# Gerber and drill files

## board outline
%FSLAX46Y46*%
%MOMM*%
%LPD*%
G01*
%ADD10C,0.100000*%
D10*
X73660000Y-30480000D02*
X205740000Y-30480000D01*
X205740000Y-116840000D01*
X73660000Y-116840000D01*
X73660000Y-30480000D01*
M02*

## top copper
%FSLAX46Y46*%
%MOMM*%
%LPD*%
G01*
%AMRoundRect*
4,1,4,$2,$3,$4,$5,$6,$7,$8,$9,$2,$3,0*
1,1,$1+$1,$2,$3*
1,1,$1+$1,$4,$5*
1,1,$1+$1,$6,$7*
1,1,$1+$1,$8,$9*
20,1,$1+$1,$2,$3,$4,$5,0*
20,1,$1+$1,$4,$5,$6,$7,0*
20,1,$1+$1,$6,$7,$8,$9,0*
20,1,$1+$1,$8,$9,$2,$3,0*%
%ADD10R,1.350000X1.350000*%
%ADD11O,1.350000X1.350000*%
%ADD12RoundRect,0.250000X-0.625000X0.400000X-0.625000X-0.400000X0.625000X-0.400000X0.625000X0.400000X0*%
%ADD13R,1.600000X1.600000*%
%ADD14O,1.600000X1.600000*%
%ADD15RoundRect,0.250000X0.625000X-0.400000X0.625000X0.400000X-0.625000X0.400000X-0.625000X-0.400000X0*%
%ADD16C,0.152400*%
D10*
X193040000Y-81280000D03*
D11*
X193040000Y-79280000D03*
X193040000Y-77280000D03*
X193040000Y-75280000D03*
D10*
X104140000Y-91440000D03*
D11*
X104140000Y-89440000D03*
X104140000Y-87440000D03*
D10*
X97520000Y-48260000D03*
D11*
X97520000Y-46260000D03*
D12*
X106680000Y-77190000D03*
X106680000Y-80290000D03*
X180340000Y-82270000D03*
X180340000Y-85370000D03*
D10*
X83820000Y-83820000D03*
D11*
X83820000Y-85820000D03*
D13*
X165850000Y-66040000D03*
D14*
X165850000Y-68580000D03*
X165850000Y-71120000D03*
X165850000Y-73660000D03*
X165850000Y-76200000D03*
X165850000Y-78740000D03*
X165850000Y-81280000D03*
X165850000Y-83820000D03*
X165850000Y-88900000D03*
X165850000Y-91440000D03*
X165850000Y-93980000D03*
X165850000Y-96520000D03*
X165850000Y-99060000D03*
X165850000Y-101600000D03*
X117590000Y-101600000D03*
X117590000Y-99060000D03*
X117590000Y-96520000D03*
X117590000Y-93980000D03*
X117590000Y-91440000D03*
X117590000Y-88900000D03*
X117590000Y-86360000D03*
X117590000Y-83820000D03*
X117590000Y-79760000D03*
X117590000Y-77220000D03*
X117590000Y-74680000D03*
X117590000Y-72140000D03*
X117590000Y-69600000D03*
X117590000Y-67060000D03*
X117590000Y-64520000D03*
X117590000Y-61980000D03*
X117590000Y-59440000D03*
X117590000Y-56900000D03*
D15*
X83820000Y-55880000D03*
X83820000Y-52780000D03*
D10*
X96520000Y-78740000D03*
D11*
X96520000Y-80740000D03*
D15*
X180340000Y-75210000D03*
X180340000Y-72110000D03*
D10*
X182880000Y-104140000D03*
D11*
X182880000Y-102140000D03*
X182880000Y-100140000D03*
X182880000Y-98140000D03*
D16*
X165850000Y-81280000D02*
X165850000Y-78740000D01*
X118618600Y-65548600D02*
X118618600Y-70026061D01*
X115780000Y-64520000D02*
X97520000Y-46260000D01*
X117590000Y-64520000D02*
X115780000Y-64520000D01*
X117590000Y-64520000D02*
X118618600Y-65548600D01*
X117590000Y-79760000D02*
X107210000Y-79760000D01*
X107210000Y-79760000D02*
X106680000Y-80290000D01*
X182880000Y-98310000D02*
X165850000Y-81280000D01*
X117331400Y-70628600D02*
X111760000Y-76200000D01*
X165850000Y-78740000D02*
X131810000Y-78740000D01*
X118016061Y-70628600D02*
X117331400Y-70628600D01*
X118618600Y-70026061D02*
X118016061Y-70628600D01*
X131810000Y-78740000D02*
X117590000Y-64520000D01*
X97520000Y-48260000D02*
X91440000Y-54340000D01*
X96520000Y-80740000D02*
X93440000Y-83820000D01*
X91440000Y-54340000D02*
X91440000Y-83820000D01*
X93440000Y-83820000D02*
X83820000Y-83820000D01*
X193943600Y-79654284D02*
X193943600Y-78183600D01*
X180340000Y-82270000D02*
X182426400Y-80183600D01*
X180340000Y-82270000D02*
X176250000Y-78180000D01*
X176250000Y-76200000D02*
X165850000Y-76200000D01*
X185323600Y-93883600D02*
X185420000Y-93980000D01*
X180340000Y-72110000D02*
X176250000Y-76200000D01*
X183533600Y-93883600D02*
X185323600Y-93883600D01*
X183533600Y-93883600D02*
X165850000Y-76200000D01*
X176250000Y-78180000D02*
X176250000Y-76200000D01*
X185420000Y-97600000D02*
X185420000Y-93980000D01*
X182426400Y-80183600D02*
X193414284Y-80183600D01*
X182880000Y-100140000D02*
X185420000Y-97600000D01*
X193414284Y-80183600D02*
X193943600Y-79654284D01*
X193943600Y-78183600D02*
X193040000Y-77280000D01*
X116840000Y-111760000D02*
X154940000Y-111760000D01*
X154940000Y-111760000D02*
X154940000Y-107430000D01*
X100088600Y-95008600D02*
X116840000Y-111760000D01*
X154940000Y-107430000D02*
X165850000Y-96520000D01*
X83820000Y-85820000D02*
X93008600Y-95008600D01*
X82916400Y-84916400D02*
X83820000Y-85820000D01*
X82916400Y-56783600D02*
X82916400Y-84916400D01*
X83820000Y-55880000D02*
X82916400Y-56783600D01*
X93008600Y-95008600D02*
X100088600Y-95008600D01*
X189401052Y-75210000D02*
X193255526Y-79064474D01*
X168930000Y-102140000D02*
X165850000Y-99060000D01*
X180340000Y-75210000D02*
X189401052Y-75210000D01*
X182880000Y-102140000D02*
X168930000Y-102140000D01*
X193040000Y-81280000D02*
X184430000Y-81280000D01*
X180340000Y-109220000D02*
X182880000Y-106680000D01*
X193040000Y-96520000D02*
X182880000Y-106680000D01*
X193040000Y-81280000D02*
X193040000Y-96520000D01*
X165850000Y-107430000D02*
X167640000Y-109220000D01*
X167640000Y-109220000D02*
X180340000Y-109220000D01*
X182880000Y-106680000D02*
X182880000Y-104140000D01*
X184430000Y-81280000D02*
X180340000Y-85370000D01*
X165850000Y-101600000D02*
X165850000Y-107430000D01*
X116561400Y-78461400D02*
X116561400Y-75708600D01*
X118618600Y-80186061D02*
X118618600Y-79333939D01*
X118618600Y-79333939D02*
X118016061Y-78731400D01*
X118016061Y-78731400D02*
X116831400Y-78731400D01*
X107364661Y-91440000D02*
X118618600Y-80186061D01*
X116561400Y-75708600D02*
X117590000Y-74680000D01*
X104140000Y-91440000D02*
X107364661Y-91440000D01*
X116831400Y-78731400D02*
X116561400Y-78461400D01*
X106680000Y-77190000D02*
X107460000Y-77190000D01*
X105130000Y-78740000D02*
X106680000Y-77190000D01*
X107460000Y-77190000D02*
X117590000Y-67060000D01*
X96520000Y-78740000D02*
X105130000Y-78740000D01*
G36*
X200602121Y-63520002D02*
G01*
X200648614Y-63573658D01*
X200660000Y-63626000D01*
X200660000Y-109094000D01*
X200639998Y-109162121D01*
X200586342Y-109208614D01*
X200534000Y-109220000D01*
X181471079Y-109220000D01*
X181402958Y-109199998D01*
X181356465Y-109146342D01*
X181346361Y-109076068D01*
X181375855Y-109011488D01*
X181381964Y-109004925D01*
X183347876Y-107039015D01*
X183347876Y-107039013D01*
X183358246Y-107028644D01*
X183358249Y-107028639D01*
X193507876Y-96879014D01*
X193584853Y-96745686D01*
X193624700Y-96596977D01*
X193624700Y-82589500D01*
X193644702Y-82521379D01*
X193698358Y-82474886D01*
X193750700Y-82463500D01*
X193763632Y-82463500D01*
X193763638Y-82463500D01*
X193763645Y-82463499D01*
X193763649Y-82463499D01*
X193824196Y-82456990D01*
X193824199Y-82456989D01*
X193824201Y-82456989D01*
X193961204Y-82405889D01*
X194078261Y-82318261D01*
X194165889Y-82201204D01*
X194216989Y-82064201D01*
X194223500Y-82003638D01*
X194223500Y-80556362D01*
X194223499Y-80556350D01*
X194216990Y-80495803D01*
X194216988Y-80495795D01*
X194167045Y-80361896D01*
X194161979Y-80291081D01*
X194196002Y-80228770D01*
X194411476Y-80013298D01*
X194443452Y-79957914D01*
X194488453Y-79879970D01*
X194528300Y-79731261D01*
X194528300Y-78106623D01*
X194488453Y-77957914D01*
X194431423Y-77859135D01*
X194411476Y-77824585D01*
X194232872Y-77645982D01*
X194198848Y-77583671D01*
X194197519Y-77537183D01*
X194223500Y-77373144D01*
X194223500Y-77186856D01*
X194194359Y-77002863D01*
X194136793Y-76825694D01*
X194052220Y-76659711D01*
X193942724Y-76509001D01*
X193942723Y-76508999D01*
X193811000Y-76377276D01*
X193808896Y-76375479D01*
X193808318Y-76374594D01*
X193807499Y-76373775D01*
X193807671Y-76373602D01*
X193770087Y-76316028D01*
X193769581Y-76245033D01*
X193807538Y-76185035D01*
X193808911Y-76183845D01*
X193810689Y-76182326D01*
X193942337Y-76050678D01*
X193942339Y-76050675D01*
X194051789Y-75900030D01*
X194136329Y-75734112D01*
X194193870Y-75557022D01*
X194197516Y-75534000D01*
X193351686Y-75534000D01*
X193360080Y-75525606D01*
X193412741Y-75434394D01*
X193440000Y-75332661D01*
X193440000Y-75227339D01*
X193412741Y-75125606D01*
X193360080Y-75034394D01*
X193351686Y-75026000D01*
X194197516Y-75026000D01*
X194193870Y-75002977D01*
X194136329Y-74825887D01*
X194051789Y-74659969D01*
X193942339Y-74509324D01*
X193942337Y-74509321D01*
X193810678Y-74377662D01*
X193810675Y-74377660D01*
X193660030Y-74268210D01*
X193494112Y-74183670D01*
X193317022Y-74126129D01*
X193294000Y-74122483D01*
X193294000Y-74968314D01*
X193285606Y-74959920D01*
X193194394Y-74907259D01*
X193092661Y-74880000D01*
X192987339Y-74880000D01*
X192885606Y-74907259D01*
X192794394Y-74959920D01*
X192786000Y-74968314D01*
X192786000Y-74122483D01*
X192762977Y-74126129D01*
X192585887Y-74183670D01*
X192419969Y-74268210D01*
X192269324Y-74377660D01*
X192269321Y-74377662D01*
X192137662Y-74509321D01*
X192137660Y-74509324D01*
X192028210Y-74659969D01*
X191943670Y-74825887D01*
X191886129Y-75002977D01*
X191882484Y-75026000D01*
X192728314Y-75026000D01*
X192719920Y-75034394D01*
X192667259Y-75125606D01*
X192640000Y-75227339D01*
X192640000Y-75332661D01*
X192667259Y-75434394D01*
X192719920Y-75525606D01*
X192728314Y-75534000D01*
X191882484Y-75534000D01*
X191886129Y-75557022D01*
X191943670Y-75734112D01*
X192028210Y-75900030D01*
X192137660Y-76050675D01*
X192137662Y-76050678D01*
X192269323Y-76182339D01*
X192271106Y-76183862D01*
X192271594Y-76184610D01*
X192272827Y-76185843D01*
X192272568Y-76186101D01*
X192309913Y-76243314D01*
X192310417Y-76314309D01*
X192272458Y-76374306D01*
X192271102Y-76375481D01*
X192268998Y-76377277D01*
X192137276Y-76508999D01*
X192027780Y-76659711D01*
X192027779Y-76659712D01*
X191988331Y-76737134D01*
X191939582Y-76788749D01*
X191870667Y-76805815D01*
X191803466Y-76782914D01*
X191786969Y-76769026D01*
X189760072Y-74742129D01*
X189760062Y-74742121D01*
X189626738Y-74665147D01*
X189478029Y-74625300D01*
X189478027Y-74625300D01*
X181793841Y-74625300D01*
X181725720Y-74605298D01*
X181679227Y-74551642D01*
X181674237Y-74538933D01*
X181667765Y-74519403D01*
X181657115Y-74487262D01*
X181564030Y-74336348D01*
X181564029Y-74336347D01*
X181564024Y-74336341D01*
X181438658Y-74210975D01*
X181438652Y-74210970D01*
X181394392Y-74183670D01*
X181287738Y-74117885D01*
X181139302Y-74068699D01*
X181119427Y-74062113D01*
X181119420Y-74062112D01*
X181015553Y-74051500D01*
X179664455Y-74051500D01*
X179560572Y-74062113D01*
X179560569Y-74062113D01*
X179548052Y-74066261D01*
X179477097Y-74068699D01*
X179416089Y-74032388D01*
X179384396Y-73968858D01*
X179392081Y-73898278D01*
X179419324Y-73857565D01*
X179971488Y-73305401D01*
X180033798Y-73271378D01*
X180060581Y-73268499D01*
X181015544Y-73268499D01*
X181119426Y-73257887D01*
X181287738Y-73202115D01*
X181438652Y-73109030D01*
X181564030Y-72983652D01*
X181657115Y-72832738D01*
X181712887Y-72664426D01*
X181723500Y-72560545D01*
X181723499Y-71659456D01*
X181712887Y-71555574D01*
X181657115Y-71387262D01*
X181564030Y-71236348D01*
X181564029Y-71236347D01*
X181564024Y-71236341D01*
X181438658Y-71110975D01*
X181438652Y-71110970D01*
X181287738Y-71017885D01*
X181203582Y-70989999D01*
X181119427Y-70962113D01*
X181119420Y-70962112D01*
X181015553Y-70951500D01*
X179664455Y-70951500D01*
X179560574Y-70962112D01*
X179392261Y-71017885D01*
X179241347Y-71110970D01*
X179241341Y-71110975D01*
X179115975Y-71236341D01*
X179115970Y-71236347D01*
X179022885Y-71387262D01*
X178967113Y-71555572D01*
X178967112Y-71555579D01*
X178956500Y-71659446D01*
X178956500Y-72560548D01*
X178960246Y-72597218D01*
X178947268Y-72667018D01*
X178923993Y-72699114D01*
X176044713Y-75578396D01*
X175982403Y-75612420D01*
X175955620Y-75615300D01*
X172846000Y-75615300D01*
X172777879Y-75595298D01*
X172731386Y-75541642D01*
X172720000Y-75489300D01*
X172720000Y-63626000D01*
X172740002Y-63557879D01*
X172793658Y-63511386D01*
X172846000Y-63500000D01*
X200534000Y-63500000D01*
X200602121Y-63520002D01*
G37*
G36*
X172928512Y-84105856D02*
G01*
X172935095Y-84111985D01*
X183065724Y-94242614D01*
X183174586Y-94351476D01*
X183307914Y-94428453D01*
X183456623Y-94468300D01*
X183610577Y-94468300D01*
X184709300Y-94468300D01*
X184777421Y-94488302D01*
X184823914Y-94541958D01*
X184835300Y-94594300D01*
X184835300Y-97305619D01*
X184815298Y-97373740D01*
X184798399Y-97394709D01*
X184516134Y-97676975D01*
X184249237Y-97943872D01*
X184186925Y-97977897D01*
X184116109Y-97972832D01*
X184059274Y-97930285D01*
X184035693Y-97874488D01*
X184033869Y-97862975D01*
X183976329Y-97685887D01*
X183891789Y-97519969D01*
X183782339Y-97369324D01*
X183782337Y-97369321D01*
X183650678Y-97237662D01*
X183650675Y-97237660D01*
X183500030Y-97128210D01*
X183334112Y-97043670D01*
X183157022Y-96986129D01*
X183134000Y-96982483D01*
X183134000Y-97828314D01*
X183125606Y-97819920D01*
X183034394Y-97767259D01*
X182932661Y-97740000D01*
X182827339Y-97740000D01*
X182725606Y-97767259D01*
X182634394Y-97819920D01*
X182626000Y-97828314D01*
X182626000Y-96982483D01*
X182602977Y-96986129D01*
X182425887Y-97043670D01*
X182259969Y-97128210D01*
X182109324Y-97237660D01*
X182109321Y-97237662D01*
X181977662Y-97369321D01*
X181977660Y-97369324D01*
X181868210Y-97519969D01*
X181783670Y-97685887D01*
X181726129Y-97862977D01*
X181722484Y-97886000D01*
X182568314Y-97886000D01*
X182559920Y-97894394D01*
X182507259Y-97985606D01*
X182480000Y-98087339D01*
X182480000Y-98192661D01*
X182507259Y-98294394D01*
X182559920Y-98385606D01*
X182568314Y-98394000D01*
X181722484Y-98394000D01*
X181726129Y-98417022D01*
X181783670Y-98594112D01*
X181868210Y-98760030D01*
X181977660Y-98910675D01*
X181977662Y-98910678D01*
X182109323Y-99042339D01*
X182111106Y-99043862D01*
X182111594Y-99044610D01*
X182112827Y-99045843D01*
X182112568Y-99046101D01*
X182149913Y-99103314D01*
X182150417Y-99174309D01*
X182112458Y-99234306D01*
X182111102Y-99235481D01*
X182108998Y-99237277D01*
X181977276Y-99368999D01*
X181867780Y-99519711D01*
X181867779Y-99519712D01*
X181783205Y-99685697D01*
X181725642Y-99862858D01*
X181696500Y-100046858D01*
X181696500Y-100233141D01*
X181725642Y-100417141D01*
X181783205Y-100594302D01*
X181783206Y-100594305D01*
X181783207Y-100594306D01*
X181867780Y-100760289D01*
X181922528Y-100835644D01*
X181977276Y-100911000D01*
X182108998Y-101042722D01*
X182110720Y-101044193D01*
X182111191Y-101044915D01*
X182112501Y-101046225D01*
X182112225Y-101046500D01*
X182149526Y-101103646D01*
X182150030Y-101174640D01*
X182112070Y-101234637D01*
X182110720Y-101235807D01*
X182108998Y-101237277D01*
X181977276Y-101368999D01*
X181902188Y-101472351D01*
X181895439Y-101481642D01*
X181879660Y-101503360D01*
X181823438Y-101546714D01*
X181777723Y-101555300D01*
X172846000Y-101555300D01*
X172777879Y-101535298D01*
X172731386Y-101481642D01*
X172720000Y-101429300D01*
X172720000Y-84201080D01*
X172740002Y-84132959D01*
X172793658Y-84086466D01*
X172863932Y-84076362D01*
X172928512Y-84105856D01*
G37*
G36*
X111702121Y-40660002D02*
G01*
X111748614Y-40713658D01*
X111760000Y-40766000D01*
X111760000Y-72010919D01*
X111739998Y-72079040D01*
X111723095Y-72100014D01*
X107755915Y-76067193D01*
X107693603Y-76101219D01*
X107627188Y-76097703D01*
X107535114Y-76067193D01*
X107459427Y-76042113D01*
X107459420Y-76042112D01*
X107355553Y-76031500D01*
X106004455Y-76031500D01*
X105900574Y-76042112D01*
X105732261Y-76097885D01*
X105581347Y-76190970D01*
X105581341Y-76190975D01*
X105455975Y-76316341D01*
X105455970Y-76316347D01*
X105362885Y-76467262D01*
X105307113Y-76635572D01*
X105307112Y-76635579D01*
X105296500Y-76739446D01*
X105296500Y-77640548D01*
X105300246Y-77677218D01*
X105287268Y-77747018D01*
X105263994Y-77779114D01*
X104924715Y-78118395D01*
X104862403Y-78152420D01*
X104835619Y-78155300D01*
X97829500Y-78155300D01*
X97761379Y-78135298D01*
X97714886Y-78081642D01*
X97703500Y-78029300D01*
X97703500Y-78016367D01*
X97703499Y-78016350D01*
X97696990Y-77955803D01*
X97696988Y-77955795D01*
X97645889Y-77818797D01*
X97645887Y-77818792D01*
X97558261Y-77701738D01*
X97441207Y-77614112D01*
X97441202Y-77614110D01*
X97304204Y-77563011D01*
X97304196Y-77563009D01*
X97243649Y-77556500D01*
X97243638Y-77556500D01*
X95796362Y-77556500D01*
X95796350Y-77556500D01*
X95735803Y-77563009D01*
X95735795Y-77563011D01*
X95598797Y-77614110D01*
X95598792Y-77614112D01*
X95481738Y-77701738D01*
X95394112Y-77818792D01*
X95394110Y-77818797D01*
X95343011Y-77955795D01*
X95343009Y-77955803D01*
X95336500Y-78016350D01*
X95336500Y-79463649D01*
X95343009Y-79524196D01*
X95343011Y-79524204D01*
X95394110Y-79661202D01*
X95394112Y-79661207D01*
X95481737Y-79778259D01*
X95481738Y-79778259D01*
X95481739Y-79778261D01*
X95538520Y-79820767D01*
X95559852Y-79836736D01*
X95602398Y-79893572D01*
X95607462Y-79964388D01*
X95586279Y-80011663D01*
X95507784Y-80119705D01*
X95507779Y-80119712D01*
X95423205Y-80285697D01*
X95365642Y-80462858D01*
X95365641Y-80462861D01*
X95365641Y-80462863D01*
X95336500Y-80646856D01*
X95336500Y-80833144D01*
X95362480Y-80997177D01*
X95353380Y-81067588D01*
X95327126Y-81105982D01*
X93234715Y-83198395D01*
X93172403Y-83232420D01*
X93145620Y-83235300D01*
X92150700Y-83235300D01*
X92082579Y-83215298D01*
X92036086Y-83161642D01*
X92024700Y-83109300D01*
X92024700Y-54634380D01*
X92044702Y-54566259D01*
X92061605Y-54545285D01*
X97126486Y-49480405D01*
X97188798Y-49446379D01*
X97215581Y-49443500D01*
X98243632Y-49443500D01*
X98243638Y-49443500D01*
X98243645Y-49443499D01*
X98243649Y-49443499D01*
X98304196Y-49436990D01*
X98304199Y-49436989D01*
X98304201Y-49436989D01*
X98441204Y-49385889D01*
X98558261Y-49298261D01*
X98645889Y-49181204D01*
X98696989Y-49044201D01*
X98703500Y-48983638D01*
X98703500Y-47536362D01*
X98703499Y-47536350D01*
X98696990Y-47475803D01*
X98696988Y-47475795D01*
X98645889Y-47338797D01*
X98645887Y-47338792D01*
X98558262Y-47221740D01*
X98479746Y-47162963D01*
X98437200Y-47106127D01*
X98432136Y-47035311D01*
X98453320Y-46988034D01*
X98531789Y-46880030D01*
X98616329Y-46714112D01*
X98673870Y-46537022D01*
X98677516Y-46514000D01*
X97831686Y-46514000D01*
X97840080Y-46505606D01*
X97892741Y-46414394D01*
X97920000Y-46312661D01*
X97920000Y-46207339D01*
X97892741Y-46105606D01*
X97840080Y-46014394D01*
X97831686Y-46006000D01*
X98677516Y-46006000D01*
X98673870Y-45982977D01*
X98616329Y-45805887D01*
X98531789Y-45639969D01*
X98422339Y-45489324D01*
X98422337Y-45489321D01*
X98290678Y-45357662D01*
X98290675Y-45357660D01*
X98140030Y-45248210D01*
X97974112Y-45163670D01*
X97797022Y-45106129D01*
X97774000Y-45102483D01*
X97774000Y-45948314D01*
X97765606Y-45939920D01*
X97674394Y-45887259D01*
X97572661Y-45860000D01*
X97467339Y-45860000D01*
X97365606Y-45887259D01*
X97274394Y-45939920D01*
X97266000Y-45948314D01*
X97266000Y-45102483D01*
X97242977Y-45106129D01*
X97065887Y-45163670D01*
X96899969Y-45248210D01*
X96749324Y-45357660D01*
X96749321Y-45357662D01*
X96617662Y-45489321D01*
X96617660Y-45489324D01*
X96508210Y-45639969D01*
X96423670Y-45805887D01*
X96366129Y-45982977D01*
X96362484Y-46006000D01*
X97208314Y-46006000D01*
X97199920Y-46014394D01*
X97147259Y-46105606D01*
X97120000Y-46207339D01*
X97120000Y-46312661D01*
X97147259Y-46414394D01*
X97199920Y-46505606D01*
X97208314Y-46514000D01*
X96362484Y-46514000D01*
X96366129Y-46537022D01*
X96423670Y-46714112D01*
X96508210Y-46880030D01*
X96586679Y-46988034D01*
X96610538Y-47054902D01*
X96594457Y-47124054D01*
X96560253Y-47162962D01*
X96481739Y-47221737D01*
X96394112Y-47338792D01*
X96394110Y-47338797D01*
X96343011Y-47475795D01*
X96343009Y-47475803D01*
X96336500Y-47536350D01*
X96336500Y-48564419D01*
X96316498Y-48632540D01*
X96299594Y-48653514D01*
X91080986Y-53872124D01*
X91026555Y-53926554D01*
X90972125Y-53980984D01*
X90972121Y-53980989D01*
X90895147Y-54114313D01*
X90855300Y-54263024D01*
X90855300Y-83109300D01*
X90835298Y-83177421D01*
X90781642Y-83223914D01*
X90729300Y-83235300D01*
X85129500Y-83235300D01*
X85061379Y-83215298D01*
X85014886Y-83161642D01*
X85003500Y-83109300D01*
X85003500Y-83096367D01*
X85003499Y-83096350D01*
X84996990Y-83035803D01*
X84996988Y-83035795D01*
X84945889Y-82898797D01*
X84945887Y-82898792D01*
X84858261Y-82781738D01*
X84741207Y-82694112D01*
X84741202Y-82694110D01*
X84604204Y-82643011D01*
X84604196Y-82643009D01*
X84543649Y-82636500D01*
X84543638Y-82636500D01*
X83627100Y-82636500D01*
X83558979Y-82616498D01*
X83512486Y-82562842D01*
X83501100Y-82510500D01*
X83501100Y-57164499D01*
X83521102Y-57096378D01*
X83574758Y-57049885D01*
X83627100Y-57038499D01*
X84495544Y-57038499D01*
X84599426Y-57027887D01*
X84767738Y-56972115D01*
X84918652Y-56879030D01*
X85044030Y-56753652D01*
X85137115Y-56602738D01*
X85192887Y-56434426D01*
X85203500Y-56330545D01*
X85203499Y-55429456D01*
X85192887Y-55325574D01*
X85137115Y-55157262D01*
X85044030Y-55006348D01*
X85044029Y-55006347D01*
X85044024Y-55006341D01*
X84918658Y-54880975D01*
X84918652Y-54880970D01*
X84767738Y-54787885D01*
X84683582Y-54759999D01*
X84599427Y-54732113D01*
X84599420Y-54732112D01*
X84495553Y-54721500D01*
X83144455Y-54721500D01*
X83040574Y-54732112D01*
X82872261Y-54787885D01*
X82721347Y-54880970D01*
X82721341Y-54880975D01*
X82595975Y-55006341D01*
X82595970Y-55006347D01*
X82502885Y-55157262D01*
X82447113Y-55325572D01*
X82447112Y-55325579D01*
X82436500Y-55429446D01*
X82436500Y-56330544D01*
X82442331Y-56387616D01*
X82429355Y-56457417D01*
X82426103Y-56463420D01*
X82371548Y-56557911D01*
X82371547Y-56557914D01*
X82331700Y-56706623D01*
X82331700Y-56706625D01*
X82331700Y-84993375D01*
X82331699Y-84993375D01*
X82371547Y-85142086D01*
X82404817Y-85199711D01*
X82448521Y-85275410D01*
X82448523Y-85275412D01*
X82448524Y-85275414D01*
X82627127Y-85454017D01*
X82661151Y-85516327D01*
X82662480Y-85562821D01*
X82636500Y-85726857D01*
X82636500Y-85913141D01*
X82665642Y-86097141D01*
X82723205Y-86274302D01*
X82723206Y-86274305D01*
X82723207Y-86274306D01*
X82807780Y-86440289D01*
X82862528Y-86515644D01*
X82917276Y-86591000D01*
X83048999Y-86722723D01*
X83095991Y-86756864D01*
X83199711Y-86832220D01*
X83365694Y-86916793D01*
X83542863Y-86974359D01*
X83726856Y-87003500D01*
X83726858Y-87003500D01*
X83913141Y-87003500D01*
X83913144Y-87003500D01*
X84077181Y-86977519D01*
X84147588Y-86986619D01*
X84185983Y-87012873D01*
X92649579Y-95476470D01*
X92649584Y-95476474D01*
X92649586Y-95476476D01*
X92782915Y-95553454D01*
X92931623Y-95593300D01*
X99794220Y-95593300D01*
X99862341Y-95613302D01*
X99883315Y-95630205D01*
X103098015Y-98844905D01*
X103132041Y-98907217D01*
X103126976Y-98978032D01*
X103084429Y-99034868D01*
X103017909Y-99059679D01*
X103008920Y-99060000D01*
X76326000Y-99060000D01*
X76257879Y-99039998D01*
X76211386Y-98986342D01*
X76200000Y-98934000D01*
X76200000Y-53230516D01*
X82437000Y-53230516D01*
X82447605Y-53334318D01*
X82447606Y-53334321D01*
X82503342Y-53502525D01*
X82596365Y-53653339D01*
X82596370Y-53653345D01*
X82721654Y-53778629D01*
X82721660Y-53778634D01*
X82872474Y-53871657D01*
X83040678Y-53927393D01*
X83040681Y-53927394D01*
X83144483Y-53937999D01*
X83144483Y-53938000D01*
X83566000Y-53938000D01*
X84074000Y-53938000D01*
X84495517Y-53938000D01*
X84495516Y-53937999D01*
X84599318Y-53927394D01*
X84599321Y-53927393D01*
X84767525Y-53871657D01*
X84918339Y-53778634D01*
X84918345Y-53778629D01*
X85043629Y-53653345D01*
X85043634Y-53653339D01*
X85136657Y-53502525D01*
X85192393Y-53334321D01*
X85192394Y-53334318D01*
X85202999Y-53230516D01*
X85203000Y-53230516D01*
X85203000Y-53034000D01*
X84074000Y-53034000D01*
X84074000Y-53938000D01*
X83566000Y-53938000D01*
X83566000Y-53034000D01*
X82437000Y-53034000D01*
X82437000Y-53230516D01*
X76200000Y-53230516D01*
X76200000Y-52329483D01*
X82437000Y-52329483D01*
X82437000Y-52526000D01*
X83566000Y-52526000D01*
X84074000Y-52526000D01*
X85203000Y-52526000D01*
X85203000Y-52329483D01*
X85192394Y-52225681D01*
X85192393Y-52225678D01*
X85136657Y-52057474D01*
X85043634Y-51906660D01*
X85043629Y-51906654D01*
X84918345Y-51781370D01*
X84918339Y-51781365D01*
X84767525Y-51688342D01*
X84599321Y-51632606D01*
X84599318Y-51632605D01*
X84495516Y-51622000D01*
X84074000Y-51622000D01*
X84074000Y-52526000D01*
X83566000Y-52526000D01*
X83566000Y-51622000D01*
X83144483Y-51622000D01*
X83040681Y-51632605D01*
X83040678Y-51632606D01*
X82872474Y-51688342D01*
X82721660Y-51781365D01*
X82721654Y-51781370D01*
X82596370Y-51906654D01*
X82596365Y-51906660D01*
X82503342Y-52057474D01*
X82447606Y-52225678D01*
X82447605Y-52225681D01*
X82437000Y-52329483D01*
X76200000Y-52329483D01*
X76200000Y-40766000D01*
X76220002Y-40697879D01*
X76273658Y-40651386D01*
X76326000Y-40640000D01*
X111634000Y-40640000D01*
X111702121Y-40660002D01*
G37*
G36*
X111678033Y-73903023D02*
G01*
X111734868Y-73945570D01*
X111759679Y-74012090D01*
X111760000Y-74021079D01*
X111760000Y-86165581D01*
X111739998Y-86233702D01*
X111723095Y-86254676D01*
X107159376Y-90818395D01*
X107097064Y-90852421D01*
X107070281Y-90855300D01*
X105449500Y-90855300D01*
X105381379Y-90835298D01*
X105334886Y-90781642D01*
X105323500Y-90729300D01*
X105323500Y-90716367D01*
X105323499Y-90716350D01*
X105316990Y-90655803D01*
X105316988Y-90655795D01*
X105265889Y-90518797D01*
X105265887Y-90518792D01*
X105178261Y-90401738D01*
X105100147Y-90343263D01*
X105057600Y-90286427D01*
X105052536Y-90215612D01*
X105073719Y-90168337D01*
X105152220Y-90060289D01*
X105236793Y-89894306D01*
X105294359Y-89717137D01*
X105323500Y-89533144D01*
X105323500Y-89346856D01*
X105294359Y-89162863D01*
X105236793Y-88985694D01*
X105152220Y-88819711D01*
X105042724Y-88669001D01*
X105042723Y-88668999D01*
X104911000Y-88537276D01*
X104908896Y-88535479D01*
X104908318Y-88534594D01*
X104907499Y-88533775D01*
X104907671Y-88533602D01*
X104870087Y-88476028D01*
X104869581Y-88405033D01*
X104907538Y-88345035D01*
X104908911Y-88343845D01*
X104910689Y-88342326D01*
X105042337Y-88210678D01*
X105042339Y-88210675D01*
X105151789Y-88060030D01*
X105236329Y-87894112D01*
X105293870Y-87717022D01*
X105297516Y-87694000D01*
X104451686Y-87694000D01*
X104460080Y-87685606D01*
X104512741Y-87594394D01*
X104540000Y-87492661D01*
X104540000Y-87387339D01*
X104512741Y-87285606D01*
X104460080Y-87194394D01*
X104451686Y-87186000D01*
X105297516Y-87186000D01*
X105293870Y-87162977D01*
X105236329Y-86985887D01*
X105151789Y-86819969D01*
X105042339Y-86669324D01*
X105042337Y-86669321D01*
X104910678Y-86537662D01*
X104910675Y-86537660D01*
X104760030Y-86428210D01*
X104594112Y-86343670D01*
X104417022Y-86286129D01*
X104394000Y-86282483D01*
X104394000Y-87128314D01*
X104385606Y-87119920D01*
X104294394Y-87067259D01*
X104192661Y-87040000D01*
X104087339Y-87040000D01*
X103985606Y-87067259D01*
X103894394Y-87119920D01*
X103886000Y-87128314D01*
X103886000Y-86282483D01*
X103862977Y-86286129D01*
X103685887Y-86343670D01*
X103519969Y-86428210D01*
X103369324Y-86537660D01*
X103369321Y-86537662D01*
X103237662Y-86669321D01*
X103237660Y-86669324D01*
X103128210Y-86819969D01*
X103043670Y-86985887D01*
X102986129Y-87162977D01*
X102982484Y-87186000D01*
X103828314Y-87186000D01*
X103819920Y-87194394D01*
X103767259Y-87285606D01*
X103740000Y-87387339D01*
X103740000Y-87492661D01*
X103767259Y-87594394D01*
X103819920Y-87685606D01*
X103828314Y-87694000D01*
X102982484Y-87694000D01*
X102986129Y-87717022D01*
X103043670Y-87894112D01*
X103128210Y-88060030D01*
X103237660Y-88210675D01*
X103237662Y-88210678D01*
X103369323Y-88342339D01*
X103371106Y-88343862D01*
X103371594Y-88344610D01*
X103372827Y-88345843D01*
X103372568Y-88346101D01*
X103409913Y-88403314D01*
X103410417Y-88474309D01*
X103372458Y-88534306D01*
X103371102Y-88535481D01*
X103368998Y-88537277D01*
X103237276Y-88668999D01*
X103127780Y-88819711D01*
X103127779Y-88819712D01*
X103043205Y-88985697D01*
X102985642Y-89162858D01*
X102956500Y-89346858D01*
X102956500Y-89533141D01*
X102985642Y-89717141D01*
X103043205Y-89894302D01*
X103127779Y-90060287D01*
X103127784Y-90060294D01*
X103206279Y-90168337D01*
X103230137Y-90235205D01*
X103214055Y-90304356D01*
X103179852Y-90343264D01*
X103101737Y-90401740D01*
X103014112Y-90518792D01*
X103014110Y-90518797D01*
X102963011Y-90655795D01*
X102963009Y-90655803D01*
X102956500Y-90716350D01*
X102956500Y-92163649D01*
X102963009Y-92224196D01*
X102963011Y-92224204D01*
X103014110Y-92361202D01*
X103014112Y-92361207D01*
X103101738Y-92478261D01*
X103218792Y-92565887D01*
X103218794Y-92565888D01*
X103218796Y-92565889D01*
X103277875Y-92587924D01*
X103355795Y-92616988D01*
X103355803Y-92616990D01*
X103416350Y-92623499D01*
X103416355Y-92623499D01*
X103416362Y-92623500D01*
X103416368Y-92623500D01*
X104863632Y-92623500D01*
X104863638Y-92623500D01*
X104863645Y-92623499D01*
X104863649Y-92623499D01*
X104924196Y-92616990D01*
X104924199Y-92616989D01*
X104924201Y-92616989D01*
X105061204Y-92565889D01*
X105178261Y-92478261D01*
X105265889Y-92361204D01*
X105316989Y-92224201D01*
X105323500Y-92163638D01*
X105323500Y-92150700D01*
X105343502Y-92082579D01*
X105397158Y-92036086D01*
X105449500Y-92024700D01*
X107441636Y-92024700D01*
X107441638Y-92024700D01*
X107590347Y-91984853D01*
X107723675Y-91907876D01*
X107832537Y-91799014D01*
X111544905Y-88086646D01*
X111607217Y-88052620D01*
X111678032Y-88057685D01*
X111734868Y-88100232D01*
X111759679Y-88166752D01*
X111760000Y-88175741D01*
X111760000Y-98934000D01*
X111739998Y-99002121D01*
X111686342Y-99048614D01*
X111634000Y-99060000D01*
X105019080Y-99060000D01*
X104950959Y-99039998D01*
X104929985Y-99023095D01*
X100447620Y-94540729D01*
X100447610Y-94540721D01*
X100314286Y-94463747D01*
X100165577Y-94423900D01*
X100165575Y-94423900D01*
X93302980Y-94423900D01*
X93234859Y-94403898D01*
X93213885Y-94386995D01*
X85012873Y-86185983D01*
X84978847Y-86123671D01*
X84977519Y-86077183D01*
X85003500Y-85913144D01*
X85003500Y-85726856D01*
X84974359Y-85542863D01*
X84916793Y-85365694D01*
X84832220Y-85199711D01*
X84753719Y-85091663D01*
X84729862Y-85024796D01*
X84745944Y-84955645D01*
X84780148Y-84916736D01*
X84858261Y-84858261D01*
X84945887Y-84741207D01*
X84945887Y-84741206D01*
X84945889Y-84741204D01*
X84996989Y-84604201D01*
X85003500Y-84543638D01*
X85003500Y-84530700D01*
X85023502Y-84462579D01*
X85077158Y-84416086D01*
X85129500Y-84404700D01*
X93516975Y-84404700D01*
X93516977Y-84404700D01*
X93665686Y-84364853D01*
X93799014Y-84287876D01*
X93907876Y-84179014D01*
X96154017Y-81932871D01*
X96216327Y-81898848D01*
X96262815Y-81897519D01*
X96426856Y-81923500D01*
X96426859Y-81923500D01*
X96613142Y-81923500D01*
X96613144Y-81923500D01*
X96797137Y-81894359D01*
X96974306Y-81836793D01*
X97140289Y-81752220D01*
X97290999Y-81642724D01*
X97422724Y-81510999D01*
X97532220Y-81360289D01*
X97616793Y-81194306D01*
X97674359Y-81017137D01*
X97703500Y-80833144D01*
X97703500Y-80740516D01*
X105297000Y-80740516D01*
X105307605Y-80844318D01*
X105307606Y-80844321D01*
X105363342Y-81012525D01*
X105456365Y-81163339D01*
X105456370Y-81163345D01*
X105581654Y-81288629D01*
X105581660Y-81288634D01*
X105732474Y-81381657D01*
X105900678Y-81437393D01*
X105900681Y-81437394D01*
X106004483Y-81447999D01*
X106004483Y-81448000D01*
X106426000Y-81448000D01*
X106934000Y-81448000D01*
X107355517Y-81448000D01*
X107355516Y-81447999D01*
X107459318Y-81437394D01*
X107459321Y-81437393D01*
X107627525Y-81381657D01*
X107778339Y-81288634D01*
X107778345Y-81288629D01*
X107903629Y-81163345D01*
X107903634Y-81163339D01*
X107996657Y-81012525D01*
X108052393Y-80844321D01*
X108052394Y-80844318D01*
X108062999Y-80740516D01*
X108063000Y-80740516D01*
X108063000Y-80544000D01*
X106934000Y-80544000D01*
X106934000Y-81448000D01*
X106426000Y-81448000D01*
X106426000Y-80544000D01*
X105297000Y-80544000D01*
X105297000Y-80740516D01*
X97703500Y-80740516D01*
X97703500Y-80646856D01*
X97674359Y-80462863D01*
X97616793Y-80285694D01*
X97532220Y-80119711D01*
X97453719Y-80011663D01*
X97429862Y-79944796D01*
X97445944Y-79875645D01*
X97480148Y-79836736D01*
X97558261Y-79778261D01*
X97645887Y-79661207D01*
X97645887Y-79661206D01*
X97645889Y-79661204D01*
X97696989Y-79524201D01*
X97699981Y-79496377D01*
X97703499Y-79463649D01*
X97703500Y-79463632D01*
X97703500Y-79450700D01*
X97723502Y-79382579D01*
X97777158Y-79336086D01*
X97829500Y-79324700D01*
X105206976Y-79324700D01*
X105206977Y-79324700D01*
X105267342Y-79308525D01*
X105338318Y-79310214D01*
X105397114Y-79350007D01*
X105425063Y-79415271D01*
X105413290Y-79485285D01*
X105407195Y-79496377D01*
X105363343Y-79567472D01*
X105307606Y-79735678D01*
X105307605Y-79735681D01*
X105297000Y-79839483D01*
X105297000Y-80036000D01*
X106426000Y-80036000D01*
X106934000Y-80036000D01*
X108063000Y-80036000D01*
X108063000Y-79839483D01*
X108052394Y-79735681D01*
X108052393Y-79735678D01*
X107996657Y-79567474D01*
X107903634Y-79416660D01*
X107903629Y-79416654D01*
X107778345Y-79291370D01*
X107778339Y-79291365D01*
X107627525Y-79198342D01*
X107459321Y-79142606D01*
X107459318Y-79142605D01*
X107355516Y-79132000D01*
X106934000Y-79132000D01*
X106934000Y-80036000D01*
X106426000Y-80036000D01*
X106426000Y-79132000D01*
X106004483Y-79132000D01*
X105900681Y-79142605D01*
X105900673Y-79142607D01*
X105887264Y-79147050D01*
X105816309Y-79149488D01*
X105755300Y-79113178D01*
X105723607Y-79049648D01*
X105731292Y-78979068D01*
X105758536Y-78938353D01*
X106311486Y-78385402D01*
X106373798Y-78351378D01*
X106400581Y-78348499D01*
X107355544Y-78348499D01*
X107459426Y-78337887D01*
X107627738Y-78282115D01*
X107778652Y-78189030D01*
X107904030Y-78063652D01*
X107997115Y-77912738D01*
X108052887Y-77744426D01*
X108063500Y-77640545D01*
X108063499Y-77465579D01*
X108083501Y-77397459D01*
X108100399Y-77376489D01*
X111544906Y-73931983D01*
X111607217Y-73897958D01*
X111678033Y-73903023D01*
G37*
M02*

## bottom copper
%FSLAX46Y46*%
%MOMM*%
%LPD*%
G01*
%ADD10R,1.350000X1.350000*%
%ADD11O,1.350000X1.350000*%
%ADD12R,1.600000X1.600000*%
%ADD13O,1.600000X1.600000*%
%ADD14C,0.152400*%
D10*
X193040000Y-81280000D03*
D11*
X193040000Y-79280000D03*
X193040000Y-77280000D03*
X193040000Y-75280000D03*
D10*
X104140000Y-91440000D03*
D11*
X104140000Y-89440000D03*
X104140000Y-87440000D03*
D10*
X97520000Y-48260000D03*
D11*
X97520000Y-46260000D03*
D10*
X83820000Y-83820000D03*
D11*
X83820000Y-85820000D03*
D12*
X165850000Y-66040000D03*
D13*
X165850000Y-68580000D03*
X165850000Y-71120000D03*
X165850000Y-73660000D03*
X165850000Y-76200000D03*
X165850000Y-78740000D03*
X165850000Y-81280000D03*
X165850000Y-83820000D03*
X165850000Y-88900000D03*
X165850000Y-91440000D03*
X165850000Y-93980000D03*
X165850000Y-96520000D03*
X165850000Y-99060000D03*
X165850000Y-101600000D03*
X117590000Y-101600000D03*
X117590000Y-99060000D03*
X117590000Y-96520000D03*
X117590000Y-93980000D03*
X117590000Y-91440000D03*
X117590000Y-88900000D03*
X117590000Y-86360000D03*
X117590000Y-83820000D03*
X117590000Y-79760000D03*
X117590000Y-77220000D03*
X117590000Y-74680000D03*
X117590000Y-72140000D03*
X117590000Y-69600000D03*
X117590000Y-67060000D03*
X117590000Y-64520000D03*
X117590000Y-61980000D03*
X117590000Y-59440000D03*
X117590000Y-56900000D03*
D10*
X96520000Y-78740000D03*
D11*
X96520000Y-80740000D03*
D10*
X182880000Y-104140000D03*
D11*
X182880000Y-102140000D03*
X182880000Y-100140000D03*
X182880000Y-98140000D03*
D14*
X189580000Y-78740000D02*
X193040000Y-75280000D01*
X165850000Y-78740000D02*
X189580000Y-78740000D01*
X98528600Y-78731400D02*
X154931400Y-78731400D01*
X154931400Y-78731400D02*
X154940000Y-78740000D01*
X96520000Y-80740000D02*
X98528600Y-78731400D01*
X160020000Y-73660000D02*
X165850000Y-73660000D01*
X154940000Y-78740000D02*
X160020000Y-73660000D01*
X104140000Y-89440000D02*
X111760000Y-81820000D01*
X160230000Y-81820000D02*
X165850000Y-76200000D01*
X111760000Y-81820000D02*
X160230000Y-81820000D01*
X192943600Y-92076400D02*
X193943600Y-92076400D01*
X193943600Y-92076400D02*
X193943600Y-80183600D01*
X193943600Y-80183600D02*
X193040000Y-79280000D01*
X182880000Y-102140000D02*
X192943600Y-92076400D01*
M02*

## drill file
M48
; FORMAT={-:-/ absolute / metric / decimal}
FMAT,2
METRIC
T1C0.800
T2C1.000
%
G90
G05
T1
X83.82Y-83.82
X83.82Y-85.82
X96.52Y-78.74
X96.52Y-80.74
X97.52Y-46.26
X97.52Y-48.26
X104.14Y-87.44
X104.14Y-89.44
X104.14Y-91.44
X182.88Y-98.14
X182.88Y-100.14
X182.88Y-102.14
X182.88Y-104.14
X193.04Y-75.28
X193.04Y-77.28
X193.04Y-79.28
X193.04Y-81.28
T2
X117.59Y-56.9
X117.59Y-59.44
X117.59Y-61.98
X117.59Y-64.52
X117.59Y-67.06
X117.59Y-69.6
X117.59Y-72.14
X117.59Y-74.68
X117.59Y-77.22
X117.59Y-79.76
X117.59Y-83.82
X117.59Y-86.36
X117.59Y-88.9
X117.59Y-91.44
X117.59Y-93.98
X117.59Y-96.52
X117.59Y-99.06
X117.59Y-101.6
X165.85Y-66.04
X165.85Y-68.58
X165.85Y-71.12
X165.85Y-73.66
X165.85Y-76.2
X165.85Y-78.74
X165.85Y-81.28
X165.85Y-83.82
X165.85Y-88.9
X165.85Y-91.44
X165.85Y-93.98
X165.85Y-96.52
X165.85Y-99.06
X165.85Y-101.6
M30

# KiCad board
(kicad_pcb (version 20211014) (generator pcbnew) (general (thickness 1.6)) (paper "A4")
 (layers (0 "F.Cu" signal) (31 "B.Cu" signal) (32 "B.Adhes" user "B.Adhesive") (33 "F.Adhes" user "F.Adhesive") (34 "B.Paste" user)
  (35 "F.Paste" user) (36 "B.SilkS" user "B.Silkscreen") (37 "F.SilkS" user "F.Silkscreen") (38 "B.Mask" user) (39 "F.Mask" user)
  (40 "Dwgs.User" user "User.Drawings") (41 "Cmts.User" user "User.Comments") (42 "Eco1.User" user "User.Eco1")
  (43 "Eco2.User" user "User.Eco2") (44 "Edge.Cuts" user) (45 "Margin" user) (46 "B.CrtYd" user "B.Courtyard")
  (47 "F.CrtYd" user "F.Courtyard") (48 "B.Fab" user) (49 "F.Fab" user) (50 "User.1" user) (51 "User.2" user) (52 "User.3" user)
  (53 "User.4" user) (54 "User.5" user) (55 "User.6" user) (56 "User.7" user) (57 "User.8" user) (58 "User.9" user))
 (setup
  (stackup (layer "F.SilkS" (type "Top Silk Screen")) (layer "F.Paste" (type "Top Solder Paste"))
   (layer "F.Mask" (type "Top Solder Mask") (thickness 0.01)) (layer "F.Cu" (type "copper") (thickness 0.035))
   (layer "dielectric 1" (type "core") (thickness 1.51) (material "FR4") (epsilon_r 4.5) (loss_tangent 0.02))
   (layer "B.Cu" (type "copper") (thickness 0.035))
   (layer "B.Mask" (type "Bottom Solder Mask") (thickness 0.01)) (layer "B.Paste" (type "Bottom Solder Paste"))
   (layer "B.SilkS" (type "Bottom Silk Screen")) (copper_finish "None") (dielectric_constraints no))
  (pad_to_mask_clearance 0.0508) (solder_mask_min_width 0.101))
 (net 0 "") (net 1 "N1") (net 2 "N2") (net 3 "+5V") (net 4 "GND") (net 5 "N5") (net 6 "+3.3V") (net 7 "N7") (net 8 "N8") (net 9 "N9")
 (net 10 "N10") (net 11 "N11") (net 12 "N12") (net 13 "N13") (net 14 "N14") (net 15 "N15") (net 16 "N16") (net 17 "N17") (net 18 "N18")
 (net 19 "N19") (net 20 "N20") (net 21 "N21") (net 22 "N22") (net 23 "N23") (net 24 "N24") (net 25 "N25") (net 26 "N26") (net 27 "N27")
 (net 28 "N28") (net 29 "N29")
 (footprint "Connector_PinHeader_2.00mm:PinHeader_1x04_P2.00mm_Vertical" (layer "F.Cu") (at 193.04 81.28 180)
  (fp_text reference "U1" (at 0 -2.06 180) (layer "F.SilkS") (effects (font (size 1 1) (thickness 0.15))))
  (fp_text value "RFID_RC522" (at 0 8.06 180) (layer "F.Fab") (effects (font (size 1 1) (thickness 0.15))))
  (pad "1" thru_hole rect (at 0 0 180) (size 1.35 1.35) (drill 0.8) (layers *.Cu *.Mask) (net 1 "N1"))
  (pad "2" thru_hole oval (at 0 2 180) (size 1.35 1.35) (drill 0.8) (layers *.Cu *.Mask) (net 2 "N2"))
  (pad "3" thru_hole oval (at 0 4 180) (size 1.35 1.35) (drill 0.8) (layers *.Cu *.Mask) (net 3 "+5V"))
  (pad "4" thru_hole oval (at 0 6 180) (size 1.35 1.35) (drill 0.8) (layers *.Cu *.Mask) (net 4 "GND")))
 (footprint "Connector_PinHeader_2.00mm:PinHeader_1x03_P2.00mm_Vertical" (layer "F.Cu") (at 104.14 91.44 180)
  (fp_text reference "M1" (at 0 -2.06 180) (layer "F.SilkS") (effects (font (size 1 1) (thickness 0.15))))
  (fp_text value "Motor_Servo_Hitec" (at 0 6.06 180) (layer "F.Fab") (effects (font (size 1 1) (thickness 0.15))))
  (pad "1" thru_hole rect (at 0 0 180) (size 1.35 1.35) (drill 0.8) (layers *.Cu *.Mask) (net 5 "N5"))
  (pad "2" thru_hole oval (at 0 2 180) (size 1.35 1.35) (drill 0.8) (layers *.Cu *.Mask) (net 3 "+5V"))
  (pad "3" thru_hole oval (at 0 4 180) (size 1.35 1.35) (drill 0.8) (layers *.Cu *.Mask) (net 4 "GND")))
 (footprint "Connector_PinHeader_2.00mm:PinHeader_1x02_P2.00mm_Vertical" (layer "F.Cu") (at 97.52 48.26 180)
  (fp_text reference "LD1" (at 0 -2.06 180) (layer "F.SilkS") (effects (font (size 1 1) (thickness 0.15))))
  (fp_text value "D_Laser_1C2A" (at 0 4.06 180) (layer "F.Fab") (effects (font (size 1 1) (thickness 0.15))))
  (pad "1" thru_hole rect (at 0 0 180) (size 1.35 1.35) (drill 0.8) (layers *.Cu *.Mask) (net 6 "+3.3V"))
  (pad "2" thru_hole oval (at 0 2 180) (size 1.35 1.35) (drill 0.8) (layers *.Cu *.Mask) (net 4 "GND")))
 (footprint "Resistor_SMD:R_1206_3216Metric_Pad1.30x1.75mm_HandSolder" (layer "F.Cu") (at 106.68 78.74 -90)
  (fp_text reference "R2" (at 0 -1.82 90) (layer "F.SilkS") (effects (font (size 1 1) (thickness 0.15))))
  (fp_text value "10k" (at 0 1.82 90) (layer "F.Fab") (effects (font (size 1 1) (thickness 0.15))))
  (pad "1" smd roundrect (at -1.55 0 270) (size 1.3 1.75) (layers "F.Cu" "F.Paste" "F.Mask") (roundrect_rratio 0.192308) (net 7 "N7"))
  (pad "2" smd roundrect (at 1.55 0 270) (size 1.3 1.75) (layers "F.Cu" "F.Paste" "F.Mask") (roundrect_rratio 0.192308) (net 4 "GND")))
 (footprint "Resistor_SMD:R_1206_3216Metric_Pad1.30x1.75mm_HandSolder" (layer "F.Cu") (at 180.34 83.82 -90)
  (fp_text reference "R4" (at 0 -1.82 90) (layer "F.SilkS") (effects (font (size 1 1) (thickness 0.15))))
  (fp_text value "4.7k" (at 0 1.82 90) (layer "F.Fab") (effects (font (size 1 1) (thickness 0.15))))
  (pad "1" smd roundrect (at -1.55 0 270) (size 1.3 1.75) (layers "F.Cu" "F.Paste" "F.Mask") (roundrect_rratio 0.192308) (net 3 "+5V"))
  (pad "2" smd roundrect (at 1.55 0 270) (size 1.3 1.75) (layers "F.Cu" "F.Paste" "F.Mask") (roundrect_rratio 0.192308) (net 1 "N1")))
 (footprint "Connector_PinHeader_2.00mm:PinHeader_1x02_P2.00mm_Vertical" (layer "F.Cu") (at 83.82 83.82)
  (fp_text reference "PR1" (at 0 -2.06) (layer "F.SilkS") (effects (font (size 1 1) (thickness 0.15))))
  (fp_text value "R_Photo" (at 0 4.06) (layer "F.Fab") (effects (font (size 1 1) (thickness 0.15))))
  (pad "1" thru_hole rect (at 0 0) (size 1.35 1.35) (drill 0.8) (layers *.Cu *.Mask) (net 6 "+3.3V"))
  (pad "2" thru_hole oval (at 0 2) (size 1.35 1.35) (drill 0.8) (layers *.Cu *.Mask) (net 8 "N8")))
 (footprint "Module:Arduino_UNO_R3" (layer "F.Cu") (at 165.85 66.04 -90)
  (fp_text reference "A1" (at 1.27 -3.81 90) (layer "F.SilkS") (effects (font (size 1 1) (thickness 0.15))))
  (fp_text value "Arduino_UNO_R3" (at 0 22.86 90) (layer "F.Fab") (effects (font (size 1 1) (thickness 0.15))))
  (pad "1" thru_hole rect (at 0 0) (size 1.6 1.6) (drill 1) (layers *.Cu *.Mask) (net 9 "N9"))
  (pad "2" thru_hole oval (at 2.54 0) (size 1.6 1.6) (drill 1) (layers *.Cu *.Mask) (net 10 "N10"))
  (pad "3" thru_hole oval (at 5.08 0) (size 1.6 1.6) (drill 1) (layers *.Cu *.Mask) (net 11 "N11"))
  (pad "4" thru_hole oval (at 7.62 0) (size 1.6 1.6) (drill 1) (layers *.Cu *.Mask) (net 6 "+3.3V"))
  (pad "5" thru_hole oval (at 10.16 0) (size 1.6 1.6) (drill 1) (layers *.Cu *.Mask) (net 3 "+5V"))
  (pad "6" thru_hole oval (at 12.7 0) (size 1.6 1.6) (drill 1) (layers *.Cu *.Mask) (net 4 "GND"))
  (pad "7" thru_hole oval (at 15.24 0) (size 1.6 1.6) (drill 1) (layers *.Cu *.Mask) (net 4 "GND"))
  (pad "8" thru_hole oval (at 17.78 0) (size 1.6 1.6) (drill 1) (layers *.Cu *.Mask) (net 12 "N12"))
  (pad "9" thru_hole oval (at 22.86 0) (size 1.6 1.6) (drill 1) (layers *.Cu *.Mask) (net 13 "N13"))
  (pad "10" thru_hole oval (at 25.4 0) (size 1.6 1.6) (drill 1) (layers *.Cu *.Mask) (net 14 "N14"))
  (pad "11" thru_hole oval (at 27.94 0) (size 1.6 1.6) (drill 1) (layers *.Cu *.Mask) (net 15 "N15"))
  (pad "12" thru_hole oval (at 30.48 0) (size 1.6 1.6) (drill 1) (layers *.Cu *.Mask) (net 8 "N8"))
  (pad "13" thru_hole oval (at 33.02 0) (size 1.6 1.6) (drill 1) (layers *.Cu *.Mask) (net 2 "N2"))
  (pad "14" thru_hole oval (at 35.56 0) (size 1.6 1.6) (drill 1) (layers *.Cu *.Mask) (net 1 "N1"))
  (pad "15" thru_hole oval (at 35.56 48.26) (size 1.6 1.6) (drill 1) (layers *.Cu *.Mask) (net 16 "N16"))
  (pad "16" thru_hole oval (at 33.02 48.26) (size 1.6 1.6) (drill 1) (layers *.Cu *.Mask) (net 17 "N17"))
  (pad "17" thru_hole oval (at 30.48 48.26) (size 1.6 1.6) (drill 1) (layers *.Cu *.Mask) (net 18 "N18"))
  (pad "18" thru_hole oval (at 27.94 48.26) (size 1.6 1.6) (drill 1) (layers *.Cu *.Mask) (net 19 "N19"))
  (pad "19" thru_hole oval (at 25.4 48.26) (size 1.6 1.6) (drill 1) (layers *.Cu *.Mask) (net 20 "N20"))
  (pad "20" thru_hole oval (at 22.86 48.26) (size 1.6 1.6) (drill 1) (layers *.Cu *.Mask) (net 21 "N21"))
  (pad "21" thru_hole oval (at 20.32 48.26) (size 1.6 1.6) (drill 1) (layers *.Cu *.Mask) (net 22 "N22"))
  (pad "22" thru_hole oval (at 17.78 48.26) (size 1.6 1.6) (drill 1) (layers *.Cu *.Mask) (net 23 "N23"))
  (pad "23" thru_hole oval (at 13.72 48.26) (size 1.6 1.6) (drill 1) (layers *.Cu *.Mask) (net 4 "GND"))
  (pad "24" thru_hole oval (at 11.18 48.26) (size 1.6 1.6) (drill 1) (layers *.Cu *.Mask) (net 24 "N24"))
  (pad "25" thru_hole oval (at 8.64 48.26) (size 1.6 1.6) (drill 1) (layers *.Cu *.Mask) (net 5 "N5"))
  (pad "26" thru_hole oval (at 6.1 48.26) (size 1.6 1.6) (drill 1) (layers *.Cu *.Mask) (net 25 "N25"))
  (pad "27" thru_hole oval (at 3.56 48.26) (size 1.6 1.6) (drill 1) (layers *.Cu *.Mask) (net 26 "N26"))
  (pad "28" thru_hole oval (at 1.02 48.26) (size 1.6 1.6) (drill 1) (layers *.Cu *.Mask) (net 7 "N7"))
  (pad "29" thru_hole oval (at -1.52 48.26) (size 1.6 1.6) (drill 1) (layers *.Cu *.Mask) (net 4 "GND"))
  (pad "30" thru_hole oval (at -4.06 48.26) (size 1.6 1.6) (drill 1) (layers *.Cu *.Mask) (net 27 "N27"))
  (pad "31" thru_hole oval (at -6.6 48.26) (size 1.6 1.6) (drill 1) (layers *.Cu *.Mask) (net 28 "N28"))
  (pad "32" thru_hole oval (at -9.14 48.26) (size 1.6 1.6) (drill 1) (layers *.Cu *.Mask) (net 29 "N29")))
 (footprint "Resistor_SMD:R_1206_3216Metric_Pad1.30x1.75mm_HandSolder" (layer "F.Cu") (at 83.82 54.33 90)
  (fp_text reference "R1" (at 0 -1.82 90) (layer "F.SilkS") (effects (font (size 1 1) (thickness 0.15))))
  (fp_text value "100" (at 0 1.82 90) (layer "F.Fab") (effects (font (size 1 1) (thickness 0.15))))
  (pad "1" smd roundrect (at -1.55 0 90) (size 1.3 1.75) (layers "F.Cu" "F.Paste" "F.Mask") (roundrect_rratio 0.192308) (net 8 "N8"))
  (pad "2" smd roundrect (at 1.55 0 90) (size 1.3 1.75) (layers "F.Cu" "F.Paste" "F.Mask") (roundrect_rratio 0.192308) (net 4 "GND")))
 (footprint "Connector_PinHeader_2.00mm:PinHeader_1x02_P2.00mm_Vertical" (layer "F.Cu") (at 96.52 78.74)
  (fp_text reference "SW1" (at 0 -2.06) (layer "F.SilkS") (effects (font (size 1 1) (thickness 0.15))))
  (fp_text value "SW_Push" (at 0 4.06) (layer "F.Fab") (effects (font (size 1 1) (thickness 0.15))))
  (pad "1" thru_hole rect (at 0 0) (size 1.35 1.35) (drill 0.8) (layers *.Cu *.Mask) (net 7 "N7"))
  (pad "2" thru_hole oval (at 0 2) (size 1.35 1.35) (drill 0.8) (layers *.Cu *.Mask) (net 6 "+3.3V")))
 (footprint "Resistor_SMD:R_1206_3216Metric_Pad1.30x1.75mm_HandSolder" (layer "F.Cu") (at 180.34 73.66 90)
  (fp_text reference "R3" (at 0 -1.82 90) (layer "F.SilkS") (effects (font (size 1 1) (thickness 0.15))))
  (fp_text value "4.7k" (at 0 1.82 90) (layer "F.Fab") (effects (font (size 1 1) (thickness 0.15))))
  (pad "1" smd roundrect (at -1.55 0 90) (size 1.3 1.75) (layers "F.Cu" "F.Paste" "F.Mask") (roundrect_rratio 0.192308) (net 2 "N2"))
  (pad "2" smd roundrect (at 1.55 0 90) (size 1.3 1.75) (layers "F.Cu" "F.Paste" "F.Mask") (roundrect_rratio 0.192308) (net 3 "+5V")))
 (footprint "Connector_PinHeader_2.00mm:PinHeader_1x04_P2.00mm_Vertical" (layer "F.Cu") (at 182.88 104.14 180)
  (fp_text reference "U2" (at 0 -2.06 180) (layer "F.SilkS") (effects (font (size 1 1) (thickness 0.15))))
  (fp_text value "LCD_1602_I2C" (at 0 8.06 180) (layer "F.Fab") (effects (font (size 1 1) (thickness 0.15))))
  (pad "1" thru_hole rect (at 0 0 180) (size 1.35 1.35) (drill 0.8) (layers *.Cu *.Mask) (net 1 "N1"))
  (pad "2" thru_hole oval (at 0 2 180) (size 1.35 1.35) (drill 0.8) (layers *.Cu *.Mask) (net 2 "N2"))
  (pad "3" thru_hole oval (at 0 4 180) (size 1.35 1.35) (drill 0.8) (layers *.Cu *.Mask) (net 3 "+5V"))
  (pad "4" thru_hole oval (at 0 6 180) (size 1.35 1.35) (drill 0.8) (layers *.Cu *.Mask) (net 4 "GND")))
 (gr_rect (start 73.66 30.48) (end 205.74 116.84) (layer "Edge.Cuts") (width 0.1) (fill none))
 (segment (start 165.85 81.28) (end 165.85 78.74) (width 0.1524) (layer "F.Cu") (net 4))
 (segment (start 118.6186 65.5486) (end 118.6186 70.026061) (width 0.1524) (layer "F.Cu") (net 4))
 (segment (start 115.78 64.52) (end 97.52 46.26) (width 0.1524) (layer "F.Cu") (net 4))
 (segment (start 117.59 64.52) (end 115.78 64.52) (width 0.1524) (layer "F.Cu") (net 4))
 (segment (start 117.59 64.52) (end 118.6186 65.5486) (width 0.1524) (layer "F.Cu") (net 4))
 (segment (start 117.59 79.76) (end 107.21 79.76) (width 0.1524) (layer "F.Cu") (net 4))
 (segment (start 107.21 79.76) (end 106.68 80.29) (width 0.1524) (layer "F.Cu") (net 4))
 (segment (start 182.88 98.31) (end 165.85 81.28) (width 0.1524) (layer "F.Cu") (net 4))
 (segment (start 117.3314 70.6286) (end 111.76 76.2) (width 0.1524) (layer "F.Cu") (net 4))
 (segment (start 165.85 78.74) (end 131.81 78.74) (width 0.1524) (layer "F.Cu") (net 4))
 (segment (start 118.016061 70.6286) (end 117.3314 70.6286) (width 0.1524) (layer "F.Cu") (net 4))
 (segment (start 118.6186 70.026061) (end 118.016061 70.6286) (width 0.1524) (layer "F.Cu") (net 4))
 (segment (start 131.81 78.74) (end 117.59 64.52) (width 0.1524) (layer "F.Cu") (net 4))
 (segment (start 189.58 78.74) (end 193.04 75.28) (width 0.1524) (layer "B.Cu") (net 4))
 (segment (start 165.85 78.74) (end 189.58 78.74) (width 0.1524) (layer "B.Cu") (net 4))
 (segment (start 97.52 48.26) (end 91.44 54.34) (width 0.1524) (layer "F.Cu") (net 6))
 (segment (start 96.52 80.74) (end 93.44 83.82) (width 0.1524) (layer "F.Cu") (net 6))
 (segment (start 91.44 54.34) (end 91.44 83.82) (width 0.1524) (layer "F.Cu") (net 6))
 (segment (start 93.44 83.82) (end 83.82 83.82) (width 0.1524) (layer "F.Cu") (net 6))
 (segment (start 98.5286 78.7314) (end 154.9314 78.7314) (width 0.1524) (layer "B.Cu") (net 6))
 (segment (start 154.9314 78.7314) (end 154.94 78.74) (width 0.1524) (layer "B.Cu") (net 6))
 (segment (start 96.52 80.74) (end 98.5286 78.7314) (width 0.1524) (layer "B.Cu") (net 6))
 (segment (start 160.02 73.66) (end 165.85 73.66) (width 0.1524) (layer "B.Cu") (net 6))
 (segment (start 154.94 78.74) (end 160.02 73.66) (width 0.1524) (layer "B.Cu") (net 6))
 (segment (start 193.9436 79.654284) (end 193.9436 78.1836) (width 0.1524) (layer "F.Cu") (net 3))
 (segment (start 180.34 82.27) (end 182.4264 80.1836) (width 0.1524) (layer "F.Cu") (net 3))
 (segment (start 180.34 82.27) (end 176.25 78.18) (width 0.1524) (layer "F.Cu") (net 3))
 (segment (start 176.25 76.2) (end 165.85 76.2) (width 0.1524) (layer "F.Cu") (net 3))
 (segment (start 185.3236 93.8836) (end 185.42 93.98) (width 0.1524) (layer "F.Cu") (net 3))
 (segment (start 180.34 72.11) (end 176.25 76.2) (width 0.1524) (layer "F.Cu") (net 3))
 (segment (start 183.5336 93.8836) (end 185.3236 93.8836) (width 0.1524) (layer "F.Cu") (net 3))
 (segment (start 183.5336 93.8836) (end 165.85 76.2) (width 0.1524) (layer "F.Cu") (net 3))
 (segment (start 176.25 78.18) (end 176.25 76.2) (width 0.1524) (layer "F.Cu") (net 3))
 (segment (start 185.42 97.6) (end 185.42 93.98) (width 0.1524) (layer "F.Cu") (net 3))
 (segment (start 182.4264 80.1836) (end 193.414284 80.1836) (width 0.1524) (layer "F.Cu") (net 3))
 (segment (start 182.88 100.14) (end 185.42 97.6) (width 0.1524) (layer "F.Cu") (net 3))
 (segment (start 193.414284 80.1836) (end 193.9436 79.654284) (width 0.1524) (layer "F.Cu") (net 3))
 (segment (start 193.9436 78.1836) (end 193.04 77.28) (width 0.1524) (layer "F.Cu") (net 3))
 (segment (start 104.14 89.44) (end 111.76 81.82) (width 0.1524) (layer "B.Cu") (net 3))
 (segment (start 160.23 81.82) (end 165.85 76.2) (width 0.1524) (layer "B.Cu") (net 3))
 (segment (start 111.76 81.82) (end 160.23 81.82) (width 0.1524) (layer "B.Cu") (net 3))
 (segment (start 116.84 111.76) (end 154.94 111.76) (width 0.1524) (layer "F.Cu") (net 8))
 (segment (start 154.94 111.76) (end 154.94 107.43) (width 0.1524) (layer "F.Cu") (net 8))
 (segment (start 100.0886 95.0086) (end 116.84 111.76) (width 0.1524) (layer "F.Cu") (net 8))
 (segment (start 154.94 107.43) (end 165.85 96.52) (width 0.1524) (layer "F.Cu") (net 8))
 (segment (start 83.82 85.82) (end 93.0086 95.0086) (width 0.1524) (layer "F.Cu") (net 8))
 (segment (start 82.9164 84.9164) (end 83.82 85.82) (width 0.1524) (layer "F.Cu") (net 8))
 (segment (start 82.9164 56.7836) (end 82.9164 84.9164) (width 0.1524) (layer "F.Cu") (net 8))
 (segment (start 83.82 55.88) (end 82.9164 56.7836) (width 0.1524) (layer "F.Cu") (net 8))
 (segment (start 93.0086 95.0086) (end 100.0886 95.0086) (width 0.1524) (layer "F.Cu") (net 8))
 (segment (start 189.401052 75.21) (end 193.255526 79.064474) (width 0.1524) (layer "F.Cu") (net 2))
 (segment (start 168.93 102.14) (end 165.85 99.06) (width 0.1524) (layer "F.Cu") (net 2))
 (segment (start 180.34 75.21) (end 189.401052 75.21) (width 0.1524) (layer "F.Cu") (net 2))
 (segment (start 182.88 102.14) (end 168.93 102.14) (width 0.1524) (layer "F.Cu") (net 2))
 (segment (start 192.9436 92.0764) (end 193.9436 92.0764) (width 0.1524) (layer "B.Cu") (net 2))
 (segment (start 193.9436 92.0764) (end 193.9436 80.1836) (width 0.1524) (layer "B.Cu") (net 2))
 (segment (start 193.9436 80.1836) (end 193.04 79.28) (width 0.1524) (layer "B.Cu") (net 2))
 (segment (start 182.88 102.14) (end 192.9436 92.0764) (width 0.1524) (layer "B.Cu") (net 2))
 (segment (start 193.04 81.28) (end 184.43 81.28) (width 0.1524) (layer "F.Cu") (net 1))
 (segment (start 180.34 109.22) (end 182.88 106.68) (width 0.1524) (layer "F.Cu") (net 1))
 (segment (start 193.04 96.52) (end 182.88 106.68) (width 0.1524) (layer "F.Cu") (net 1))
 (segment (start 193.04 81.28) (end 193.04 96.52) (width 0.1524) (layer "F.Cu") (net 1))
 (segment (start 165.85 107.43) (end 167.64 109.22) (width 0.1524) (layer "F.Cu") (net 1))
 (segment (start 167.64 109.22) (end 180.34 109.22) (width 0.1524) (layer "F.Cu") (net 1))
 (segment (start 182.88 106.68) (end 182.88 104.14) (width 0.1524) (layer "F.Cu") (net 1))
 (segment (start 184.43 81.28) (end 180.34 85.37) (width 0.1524) (layer "F.Cu") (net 1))
 (segment (start 165.85 101.6) (end 165.85 107.43) (width 0.1524) (layer "F.Cu") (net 1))
 (segment (start 116.5614 78.4614) (end 116.5614 75.7086) (width 0.1524) (layer "F.Cu") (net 5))
 (segment (start 118.6186 80.186061) (end 118.6186 79.333939) (width 0.1524) (layer "F.Cu") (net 5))
 (segment (start 118.6186 79.333939) (end 118.016061 78.7314) (width 0.1524) (layer "F.Cu") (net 5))
 (segment (start 118.016061 78.7314) (end 116.8314 78.7314) (width 0.1524) (layer "F.Cu") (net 5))
 (segment (start 107.364661 91.44) (end 118.6186 80.186061) (width 0.1524) (layer "F.Cu") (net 5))
 (segment (start 116.5614 75.7086) (end 117.59 74.68) (width 0.1524) (layer "F.Cu") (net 5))
 (segment (start 104.14 91.44) (end 107.364661 91.44) (width 0.1524) (layer "F.Cu") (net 5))
 (segment (start 116.8314 78.7314) (end 116.5614 78.4614) (width 0.1524) (layer "F.Cu") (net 5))
 (segment (start 106.68 77.19) (end 107.46 77.19) (width 0.1524) (layer "F.Cu") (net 7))
 (segment (start 105.13 78.74) (end 106.68 77.19) (width 0.1524) (layer "F.Cu") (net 7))
 (segment (start 107.46 77.19) (end 117.59 67.06) (width 0.1524) (layer "F.Cu") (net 7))
 (segment (start 96.52 78.74) (end 105.13 78.74) (width 0.1524) (layer "F.Cu") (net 7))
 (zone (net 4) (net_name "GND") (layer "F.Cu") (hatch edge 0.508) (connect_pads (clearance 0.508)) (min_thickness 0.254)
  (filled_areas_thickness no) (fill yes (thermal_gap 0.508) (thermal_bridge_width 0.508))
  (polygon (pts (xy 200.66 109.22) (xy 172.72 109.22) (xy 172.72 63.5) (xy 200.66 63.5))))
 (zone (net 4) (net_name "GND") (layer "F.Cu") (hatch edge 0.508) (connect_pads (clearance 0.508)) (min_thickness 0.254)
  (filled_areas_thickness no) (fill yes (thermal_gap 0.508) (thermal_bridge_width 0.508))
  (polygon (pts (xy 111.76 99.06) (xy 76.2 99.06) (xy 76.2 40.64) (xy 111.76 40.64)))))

